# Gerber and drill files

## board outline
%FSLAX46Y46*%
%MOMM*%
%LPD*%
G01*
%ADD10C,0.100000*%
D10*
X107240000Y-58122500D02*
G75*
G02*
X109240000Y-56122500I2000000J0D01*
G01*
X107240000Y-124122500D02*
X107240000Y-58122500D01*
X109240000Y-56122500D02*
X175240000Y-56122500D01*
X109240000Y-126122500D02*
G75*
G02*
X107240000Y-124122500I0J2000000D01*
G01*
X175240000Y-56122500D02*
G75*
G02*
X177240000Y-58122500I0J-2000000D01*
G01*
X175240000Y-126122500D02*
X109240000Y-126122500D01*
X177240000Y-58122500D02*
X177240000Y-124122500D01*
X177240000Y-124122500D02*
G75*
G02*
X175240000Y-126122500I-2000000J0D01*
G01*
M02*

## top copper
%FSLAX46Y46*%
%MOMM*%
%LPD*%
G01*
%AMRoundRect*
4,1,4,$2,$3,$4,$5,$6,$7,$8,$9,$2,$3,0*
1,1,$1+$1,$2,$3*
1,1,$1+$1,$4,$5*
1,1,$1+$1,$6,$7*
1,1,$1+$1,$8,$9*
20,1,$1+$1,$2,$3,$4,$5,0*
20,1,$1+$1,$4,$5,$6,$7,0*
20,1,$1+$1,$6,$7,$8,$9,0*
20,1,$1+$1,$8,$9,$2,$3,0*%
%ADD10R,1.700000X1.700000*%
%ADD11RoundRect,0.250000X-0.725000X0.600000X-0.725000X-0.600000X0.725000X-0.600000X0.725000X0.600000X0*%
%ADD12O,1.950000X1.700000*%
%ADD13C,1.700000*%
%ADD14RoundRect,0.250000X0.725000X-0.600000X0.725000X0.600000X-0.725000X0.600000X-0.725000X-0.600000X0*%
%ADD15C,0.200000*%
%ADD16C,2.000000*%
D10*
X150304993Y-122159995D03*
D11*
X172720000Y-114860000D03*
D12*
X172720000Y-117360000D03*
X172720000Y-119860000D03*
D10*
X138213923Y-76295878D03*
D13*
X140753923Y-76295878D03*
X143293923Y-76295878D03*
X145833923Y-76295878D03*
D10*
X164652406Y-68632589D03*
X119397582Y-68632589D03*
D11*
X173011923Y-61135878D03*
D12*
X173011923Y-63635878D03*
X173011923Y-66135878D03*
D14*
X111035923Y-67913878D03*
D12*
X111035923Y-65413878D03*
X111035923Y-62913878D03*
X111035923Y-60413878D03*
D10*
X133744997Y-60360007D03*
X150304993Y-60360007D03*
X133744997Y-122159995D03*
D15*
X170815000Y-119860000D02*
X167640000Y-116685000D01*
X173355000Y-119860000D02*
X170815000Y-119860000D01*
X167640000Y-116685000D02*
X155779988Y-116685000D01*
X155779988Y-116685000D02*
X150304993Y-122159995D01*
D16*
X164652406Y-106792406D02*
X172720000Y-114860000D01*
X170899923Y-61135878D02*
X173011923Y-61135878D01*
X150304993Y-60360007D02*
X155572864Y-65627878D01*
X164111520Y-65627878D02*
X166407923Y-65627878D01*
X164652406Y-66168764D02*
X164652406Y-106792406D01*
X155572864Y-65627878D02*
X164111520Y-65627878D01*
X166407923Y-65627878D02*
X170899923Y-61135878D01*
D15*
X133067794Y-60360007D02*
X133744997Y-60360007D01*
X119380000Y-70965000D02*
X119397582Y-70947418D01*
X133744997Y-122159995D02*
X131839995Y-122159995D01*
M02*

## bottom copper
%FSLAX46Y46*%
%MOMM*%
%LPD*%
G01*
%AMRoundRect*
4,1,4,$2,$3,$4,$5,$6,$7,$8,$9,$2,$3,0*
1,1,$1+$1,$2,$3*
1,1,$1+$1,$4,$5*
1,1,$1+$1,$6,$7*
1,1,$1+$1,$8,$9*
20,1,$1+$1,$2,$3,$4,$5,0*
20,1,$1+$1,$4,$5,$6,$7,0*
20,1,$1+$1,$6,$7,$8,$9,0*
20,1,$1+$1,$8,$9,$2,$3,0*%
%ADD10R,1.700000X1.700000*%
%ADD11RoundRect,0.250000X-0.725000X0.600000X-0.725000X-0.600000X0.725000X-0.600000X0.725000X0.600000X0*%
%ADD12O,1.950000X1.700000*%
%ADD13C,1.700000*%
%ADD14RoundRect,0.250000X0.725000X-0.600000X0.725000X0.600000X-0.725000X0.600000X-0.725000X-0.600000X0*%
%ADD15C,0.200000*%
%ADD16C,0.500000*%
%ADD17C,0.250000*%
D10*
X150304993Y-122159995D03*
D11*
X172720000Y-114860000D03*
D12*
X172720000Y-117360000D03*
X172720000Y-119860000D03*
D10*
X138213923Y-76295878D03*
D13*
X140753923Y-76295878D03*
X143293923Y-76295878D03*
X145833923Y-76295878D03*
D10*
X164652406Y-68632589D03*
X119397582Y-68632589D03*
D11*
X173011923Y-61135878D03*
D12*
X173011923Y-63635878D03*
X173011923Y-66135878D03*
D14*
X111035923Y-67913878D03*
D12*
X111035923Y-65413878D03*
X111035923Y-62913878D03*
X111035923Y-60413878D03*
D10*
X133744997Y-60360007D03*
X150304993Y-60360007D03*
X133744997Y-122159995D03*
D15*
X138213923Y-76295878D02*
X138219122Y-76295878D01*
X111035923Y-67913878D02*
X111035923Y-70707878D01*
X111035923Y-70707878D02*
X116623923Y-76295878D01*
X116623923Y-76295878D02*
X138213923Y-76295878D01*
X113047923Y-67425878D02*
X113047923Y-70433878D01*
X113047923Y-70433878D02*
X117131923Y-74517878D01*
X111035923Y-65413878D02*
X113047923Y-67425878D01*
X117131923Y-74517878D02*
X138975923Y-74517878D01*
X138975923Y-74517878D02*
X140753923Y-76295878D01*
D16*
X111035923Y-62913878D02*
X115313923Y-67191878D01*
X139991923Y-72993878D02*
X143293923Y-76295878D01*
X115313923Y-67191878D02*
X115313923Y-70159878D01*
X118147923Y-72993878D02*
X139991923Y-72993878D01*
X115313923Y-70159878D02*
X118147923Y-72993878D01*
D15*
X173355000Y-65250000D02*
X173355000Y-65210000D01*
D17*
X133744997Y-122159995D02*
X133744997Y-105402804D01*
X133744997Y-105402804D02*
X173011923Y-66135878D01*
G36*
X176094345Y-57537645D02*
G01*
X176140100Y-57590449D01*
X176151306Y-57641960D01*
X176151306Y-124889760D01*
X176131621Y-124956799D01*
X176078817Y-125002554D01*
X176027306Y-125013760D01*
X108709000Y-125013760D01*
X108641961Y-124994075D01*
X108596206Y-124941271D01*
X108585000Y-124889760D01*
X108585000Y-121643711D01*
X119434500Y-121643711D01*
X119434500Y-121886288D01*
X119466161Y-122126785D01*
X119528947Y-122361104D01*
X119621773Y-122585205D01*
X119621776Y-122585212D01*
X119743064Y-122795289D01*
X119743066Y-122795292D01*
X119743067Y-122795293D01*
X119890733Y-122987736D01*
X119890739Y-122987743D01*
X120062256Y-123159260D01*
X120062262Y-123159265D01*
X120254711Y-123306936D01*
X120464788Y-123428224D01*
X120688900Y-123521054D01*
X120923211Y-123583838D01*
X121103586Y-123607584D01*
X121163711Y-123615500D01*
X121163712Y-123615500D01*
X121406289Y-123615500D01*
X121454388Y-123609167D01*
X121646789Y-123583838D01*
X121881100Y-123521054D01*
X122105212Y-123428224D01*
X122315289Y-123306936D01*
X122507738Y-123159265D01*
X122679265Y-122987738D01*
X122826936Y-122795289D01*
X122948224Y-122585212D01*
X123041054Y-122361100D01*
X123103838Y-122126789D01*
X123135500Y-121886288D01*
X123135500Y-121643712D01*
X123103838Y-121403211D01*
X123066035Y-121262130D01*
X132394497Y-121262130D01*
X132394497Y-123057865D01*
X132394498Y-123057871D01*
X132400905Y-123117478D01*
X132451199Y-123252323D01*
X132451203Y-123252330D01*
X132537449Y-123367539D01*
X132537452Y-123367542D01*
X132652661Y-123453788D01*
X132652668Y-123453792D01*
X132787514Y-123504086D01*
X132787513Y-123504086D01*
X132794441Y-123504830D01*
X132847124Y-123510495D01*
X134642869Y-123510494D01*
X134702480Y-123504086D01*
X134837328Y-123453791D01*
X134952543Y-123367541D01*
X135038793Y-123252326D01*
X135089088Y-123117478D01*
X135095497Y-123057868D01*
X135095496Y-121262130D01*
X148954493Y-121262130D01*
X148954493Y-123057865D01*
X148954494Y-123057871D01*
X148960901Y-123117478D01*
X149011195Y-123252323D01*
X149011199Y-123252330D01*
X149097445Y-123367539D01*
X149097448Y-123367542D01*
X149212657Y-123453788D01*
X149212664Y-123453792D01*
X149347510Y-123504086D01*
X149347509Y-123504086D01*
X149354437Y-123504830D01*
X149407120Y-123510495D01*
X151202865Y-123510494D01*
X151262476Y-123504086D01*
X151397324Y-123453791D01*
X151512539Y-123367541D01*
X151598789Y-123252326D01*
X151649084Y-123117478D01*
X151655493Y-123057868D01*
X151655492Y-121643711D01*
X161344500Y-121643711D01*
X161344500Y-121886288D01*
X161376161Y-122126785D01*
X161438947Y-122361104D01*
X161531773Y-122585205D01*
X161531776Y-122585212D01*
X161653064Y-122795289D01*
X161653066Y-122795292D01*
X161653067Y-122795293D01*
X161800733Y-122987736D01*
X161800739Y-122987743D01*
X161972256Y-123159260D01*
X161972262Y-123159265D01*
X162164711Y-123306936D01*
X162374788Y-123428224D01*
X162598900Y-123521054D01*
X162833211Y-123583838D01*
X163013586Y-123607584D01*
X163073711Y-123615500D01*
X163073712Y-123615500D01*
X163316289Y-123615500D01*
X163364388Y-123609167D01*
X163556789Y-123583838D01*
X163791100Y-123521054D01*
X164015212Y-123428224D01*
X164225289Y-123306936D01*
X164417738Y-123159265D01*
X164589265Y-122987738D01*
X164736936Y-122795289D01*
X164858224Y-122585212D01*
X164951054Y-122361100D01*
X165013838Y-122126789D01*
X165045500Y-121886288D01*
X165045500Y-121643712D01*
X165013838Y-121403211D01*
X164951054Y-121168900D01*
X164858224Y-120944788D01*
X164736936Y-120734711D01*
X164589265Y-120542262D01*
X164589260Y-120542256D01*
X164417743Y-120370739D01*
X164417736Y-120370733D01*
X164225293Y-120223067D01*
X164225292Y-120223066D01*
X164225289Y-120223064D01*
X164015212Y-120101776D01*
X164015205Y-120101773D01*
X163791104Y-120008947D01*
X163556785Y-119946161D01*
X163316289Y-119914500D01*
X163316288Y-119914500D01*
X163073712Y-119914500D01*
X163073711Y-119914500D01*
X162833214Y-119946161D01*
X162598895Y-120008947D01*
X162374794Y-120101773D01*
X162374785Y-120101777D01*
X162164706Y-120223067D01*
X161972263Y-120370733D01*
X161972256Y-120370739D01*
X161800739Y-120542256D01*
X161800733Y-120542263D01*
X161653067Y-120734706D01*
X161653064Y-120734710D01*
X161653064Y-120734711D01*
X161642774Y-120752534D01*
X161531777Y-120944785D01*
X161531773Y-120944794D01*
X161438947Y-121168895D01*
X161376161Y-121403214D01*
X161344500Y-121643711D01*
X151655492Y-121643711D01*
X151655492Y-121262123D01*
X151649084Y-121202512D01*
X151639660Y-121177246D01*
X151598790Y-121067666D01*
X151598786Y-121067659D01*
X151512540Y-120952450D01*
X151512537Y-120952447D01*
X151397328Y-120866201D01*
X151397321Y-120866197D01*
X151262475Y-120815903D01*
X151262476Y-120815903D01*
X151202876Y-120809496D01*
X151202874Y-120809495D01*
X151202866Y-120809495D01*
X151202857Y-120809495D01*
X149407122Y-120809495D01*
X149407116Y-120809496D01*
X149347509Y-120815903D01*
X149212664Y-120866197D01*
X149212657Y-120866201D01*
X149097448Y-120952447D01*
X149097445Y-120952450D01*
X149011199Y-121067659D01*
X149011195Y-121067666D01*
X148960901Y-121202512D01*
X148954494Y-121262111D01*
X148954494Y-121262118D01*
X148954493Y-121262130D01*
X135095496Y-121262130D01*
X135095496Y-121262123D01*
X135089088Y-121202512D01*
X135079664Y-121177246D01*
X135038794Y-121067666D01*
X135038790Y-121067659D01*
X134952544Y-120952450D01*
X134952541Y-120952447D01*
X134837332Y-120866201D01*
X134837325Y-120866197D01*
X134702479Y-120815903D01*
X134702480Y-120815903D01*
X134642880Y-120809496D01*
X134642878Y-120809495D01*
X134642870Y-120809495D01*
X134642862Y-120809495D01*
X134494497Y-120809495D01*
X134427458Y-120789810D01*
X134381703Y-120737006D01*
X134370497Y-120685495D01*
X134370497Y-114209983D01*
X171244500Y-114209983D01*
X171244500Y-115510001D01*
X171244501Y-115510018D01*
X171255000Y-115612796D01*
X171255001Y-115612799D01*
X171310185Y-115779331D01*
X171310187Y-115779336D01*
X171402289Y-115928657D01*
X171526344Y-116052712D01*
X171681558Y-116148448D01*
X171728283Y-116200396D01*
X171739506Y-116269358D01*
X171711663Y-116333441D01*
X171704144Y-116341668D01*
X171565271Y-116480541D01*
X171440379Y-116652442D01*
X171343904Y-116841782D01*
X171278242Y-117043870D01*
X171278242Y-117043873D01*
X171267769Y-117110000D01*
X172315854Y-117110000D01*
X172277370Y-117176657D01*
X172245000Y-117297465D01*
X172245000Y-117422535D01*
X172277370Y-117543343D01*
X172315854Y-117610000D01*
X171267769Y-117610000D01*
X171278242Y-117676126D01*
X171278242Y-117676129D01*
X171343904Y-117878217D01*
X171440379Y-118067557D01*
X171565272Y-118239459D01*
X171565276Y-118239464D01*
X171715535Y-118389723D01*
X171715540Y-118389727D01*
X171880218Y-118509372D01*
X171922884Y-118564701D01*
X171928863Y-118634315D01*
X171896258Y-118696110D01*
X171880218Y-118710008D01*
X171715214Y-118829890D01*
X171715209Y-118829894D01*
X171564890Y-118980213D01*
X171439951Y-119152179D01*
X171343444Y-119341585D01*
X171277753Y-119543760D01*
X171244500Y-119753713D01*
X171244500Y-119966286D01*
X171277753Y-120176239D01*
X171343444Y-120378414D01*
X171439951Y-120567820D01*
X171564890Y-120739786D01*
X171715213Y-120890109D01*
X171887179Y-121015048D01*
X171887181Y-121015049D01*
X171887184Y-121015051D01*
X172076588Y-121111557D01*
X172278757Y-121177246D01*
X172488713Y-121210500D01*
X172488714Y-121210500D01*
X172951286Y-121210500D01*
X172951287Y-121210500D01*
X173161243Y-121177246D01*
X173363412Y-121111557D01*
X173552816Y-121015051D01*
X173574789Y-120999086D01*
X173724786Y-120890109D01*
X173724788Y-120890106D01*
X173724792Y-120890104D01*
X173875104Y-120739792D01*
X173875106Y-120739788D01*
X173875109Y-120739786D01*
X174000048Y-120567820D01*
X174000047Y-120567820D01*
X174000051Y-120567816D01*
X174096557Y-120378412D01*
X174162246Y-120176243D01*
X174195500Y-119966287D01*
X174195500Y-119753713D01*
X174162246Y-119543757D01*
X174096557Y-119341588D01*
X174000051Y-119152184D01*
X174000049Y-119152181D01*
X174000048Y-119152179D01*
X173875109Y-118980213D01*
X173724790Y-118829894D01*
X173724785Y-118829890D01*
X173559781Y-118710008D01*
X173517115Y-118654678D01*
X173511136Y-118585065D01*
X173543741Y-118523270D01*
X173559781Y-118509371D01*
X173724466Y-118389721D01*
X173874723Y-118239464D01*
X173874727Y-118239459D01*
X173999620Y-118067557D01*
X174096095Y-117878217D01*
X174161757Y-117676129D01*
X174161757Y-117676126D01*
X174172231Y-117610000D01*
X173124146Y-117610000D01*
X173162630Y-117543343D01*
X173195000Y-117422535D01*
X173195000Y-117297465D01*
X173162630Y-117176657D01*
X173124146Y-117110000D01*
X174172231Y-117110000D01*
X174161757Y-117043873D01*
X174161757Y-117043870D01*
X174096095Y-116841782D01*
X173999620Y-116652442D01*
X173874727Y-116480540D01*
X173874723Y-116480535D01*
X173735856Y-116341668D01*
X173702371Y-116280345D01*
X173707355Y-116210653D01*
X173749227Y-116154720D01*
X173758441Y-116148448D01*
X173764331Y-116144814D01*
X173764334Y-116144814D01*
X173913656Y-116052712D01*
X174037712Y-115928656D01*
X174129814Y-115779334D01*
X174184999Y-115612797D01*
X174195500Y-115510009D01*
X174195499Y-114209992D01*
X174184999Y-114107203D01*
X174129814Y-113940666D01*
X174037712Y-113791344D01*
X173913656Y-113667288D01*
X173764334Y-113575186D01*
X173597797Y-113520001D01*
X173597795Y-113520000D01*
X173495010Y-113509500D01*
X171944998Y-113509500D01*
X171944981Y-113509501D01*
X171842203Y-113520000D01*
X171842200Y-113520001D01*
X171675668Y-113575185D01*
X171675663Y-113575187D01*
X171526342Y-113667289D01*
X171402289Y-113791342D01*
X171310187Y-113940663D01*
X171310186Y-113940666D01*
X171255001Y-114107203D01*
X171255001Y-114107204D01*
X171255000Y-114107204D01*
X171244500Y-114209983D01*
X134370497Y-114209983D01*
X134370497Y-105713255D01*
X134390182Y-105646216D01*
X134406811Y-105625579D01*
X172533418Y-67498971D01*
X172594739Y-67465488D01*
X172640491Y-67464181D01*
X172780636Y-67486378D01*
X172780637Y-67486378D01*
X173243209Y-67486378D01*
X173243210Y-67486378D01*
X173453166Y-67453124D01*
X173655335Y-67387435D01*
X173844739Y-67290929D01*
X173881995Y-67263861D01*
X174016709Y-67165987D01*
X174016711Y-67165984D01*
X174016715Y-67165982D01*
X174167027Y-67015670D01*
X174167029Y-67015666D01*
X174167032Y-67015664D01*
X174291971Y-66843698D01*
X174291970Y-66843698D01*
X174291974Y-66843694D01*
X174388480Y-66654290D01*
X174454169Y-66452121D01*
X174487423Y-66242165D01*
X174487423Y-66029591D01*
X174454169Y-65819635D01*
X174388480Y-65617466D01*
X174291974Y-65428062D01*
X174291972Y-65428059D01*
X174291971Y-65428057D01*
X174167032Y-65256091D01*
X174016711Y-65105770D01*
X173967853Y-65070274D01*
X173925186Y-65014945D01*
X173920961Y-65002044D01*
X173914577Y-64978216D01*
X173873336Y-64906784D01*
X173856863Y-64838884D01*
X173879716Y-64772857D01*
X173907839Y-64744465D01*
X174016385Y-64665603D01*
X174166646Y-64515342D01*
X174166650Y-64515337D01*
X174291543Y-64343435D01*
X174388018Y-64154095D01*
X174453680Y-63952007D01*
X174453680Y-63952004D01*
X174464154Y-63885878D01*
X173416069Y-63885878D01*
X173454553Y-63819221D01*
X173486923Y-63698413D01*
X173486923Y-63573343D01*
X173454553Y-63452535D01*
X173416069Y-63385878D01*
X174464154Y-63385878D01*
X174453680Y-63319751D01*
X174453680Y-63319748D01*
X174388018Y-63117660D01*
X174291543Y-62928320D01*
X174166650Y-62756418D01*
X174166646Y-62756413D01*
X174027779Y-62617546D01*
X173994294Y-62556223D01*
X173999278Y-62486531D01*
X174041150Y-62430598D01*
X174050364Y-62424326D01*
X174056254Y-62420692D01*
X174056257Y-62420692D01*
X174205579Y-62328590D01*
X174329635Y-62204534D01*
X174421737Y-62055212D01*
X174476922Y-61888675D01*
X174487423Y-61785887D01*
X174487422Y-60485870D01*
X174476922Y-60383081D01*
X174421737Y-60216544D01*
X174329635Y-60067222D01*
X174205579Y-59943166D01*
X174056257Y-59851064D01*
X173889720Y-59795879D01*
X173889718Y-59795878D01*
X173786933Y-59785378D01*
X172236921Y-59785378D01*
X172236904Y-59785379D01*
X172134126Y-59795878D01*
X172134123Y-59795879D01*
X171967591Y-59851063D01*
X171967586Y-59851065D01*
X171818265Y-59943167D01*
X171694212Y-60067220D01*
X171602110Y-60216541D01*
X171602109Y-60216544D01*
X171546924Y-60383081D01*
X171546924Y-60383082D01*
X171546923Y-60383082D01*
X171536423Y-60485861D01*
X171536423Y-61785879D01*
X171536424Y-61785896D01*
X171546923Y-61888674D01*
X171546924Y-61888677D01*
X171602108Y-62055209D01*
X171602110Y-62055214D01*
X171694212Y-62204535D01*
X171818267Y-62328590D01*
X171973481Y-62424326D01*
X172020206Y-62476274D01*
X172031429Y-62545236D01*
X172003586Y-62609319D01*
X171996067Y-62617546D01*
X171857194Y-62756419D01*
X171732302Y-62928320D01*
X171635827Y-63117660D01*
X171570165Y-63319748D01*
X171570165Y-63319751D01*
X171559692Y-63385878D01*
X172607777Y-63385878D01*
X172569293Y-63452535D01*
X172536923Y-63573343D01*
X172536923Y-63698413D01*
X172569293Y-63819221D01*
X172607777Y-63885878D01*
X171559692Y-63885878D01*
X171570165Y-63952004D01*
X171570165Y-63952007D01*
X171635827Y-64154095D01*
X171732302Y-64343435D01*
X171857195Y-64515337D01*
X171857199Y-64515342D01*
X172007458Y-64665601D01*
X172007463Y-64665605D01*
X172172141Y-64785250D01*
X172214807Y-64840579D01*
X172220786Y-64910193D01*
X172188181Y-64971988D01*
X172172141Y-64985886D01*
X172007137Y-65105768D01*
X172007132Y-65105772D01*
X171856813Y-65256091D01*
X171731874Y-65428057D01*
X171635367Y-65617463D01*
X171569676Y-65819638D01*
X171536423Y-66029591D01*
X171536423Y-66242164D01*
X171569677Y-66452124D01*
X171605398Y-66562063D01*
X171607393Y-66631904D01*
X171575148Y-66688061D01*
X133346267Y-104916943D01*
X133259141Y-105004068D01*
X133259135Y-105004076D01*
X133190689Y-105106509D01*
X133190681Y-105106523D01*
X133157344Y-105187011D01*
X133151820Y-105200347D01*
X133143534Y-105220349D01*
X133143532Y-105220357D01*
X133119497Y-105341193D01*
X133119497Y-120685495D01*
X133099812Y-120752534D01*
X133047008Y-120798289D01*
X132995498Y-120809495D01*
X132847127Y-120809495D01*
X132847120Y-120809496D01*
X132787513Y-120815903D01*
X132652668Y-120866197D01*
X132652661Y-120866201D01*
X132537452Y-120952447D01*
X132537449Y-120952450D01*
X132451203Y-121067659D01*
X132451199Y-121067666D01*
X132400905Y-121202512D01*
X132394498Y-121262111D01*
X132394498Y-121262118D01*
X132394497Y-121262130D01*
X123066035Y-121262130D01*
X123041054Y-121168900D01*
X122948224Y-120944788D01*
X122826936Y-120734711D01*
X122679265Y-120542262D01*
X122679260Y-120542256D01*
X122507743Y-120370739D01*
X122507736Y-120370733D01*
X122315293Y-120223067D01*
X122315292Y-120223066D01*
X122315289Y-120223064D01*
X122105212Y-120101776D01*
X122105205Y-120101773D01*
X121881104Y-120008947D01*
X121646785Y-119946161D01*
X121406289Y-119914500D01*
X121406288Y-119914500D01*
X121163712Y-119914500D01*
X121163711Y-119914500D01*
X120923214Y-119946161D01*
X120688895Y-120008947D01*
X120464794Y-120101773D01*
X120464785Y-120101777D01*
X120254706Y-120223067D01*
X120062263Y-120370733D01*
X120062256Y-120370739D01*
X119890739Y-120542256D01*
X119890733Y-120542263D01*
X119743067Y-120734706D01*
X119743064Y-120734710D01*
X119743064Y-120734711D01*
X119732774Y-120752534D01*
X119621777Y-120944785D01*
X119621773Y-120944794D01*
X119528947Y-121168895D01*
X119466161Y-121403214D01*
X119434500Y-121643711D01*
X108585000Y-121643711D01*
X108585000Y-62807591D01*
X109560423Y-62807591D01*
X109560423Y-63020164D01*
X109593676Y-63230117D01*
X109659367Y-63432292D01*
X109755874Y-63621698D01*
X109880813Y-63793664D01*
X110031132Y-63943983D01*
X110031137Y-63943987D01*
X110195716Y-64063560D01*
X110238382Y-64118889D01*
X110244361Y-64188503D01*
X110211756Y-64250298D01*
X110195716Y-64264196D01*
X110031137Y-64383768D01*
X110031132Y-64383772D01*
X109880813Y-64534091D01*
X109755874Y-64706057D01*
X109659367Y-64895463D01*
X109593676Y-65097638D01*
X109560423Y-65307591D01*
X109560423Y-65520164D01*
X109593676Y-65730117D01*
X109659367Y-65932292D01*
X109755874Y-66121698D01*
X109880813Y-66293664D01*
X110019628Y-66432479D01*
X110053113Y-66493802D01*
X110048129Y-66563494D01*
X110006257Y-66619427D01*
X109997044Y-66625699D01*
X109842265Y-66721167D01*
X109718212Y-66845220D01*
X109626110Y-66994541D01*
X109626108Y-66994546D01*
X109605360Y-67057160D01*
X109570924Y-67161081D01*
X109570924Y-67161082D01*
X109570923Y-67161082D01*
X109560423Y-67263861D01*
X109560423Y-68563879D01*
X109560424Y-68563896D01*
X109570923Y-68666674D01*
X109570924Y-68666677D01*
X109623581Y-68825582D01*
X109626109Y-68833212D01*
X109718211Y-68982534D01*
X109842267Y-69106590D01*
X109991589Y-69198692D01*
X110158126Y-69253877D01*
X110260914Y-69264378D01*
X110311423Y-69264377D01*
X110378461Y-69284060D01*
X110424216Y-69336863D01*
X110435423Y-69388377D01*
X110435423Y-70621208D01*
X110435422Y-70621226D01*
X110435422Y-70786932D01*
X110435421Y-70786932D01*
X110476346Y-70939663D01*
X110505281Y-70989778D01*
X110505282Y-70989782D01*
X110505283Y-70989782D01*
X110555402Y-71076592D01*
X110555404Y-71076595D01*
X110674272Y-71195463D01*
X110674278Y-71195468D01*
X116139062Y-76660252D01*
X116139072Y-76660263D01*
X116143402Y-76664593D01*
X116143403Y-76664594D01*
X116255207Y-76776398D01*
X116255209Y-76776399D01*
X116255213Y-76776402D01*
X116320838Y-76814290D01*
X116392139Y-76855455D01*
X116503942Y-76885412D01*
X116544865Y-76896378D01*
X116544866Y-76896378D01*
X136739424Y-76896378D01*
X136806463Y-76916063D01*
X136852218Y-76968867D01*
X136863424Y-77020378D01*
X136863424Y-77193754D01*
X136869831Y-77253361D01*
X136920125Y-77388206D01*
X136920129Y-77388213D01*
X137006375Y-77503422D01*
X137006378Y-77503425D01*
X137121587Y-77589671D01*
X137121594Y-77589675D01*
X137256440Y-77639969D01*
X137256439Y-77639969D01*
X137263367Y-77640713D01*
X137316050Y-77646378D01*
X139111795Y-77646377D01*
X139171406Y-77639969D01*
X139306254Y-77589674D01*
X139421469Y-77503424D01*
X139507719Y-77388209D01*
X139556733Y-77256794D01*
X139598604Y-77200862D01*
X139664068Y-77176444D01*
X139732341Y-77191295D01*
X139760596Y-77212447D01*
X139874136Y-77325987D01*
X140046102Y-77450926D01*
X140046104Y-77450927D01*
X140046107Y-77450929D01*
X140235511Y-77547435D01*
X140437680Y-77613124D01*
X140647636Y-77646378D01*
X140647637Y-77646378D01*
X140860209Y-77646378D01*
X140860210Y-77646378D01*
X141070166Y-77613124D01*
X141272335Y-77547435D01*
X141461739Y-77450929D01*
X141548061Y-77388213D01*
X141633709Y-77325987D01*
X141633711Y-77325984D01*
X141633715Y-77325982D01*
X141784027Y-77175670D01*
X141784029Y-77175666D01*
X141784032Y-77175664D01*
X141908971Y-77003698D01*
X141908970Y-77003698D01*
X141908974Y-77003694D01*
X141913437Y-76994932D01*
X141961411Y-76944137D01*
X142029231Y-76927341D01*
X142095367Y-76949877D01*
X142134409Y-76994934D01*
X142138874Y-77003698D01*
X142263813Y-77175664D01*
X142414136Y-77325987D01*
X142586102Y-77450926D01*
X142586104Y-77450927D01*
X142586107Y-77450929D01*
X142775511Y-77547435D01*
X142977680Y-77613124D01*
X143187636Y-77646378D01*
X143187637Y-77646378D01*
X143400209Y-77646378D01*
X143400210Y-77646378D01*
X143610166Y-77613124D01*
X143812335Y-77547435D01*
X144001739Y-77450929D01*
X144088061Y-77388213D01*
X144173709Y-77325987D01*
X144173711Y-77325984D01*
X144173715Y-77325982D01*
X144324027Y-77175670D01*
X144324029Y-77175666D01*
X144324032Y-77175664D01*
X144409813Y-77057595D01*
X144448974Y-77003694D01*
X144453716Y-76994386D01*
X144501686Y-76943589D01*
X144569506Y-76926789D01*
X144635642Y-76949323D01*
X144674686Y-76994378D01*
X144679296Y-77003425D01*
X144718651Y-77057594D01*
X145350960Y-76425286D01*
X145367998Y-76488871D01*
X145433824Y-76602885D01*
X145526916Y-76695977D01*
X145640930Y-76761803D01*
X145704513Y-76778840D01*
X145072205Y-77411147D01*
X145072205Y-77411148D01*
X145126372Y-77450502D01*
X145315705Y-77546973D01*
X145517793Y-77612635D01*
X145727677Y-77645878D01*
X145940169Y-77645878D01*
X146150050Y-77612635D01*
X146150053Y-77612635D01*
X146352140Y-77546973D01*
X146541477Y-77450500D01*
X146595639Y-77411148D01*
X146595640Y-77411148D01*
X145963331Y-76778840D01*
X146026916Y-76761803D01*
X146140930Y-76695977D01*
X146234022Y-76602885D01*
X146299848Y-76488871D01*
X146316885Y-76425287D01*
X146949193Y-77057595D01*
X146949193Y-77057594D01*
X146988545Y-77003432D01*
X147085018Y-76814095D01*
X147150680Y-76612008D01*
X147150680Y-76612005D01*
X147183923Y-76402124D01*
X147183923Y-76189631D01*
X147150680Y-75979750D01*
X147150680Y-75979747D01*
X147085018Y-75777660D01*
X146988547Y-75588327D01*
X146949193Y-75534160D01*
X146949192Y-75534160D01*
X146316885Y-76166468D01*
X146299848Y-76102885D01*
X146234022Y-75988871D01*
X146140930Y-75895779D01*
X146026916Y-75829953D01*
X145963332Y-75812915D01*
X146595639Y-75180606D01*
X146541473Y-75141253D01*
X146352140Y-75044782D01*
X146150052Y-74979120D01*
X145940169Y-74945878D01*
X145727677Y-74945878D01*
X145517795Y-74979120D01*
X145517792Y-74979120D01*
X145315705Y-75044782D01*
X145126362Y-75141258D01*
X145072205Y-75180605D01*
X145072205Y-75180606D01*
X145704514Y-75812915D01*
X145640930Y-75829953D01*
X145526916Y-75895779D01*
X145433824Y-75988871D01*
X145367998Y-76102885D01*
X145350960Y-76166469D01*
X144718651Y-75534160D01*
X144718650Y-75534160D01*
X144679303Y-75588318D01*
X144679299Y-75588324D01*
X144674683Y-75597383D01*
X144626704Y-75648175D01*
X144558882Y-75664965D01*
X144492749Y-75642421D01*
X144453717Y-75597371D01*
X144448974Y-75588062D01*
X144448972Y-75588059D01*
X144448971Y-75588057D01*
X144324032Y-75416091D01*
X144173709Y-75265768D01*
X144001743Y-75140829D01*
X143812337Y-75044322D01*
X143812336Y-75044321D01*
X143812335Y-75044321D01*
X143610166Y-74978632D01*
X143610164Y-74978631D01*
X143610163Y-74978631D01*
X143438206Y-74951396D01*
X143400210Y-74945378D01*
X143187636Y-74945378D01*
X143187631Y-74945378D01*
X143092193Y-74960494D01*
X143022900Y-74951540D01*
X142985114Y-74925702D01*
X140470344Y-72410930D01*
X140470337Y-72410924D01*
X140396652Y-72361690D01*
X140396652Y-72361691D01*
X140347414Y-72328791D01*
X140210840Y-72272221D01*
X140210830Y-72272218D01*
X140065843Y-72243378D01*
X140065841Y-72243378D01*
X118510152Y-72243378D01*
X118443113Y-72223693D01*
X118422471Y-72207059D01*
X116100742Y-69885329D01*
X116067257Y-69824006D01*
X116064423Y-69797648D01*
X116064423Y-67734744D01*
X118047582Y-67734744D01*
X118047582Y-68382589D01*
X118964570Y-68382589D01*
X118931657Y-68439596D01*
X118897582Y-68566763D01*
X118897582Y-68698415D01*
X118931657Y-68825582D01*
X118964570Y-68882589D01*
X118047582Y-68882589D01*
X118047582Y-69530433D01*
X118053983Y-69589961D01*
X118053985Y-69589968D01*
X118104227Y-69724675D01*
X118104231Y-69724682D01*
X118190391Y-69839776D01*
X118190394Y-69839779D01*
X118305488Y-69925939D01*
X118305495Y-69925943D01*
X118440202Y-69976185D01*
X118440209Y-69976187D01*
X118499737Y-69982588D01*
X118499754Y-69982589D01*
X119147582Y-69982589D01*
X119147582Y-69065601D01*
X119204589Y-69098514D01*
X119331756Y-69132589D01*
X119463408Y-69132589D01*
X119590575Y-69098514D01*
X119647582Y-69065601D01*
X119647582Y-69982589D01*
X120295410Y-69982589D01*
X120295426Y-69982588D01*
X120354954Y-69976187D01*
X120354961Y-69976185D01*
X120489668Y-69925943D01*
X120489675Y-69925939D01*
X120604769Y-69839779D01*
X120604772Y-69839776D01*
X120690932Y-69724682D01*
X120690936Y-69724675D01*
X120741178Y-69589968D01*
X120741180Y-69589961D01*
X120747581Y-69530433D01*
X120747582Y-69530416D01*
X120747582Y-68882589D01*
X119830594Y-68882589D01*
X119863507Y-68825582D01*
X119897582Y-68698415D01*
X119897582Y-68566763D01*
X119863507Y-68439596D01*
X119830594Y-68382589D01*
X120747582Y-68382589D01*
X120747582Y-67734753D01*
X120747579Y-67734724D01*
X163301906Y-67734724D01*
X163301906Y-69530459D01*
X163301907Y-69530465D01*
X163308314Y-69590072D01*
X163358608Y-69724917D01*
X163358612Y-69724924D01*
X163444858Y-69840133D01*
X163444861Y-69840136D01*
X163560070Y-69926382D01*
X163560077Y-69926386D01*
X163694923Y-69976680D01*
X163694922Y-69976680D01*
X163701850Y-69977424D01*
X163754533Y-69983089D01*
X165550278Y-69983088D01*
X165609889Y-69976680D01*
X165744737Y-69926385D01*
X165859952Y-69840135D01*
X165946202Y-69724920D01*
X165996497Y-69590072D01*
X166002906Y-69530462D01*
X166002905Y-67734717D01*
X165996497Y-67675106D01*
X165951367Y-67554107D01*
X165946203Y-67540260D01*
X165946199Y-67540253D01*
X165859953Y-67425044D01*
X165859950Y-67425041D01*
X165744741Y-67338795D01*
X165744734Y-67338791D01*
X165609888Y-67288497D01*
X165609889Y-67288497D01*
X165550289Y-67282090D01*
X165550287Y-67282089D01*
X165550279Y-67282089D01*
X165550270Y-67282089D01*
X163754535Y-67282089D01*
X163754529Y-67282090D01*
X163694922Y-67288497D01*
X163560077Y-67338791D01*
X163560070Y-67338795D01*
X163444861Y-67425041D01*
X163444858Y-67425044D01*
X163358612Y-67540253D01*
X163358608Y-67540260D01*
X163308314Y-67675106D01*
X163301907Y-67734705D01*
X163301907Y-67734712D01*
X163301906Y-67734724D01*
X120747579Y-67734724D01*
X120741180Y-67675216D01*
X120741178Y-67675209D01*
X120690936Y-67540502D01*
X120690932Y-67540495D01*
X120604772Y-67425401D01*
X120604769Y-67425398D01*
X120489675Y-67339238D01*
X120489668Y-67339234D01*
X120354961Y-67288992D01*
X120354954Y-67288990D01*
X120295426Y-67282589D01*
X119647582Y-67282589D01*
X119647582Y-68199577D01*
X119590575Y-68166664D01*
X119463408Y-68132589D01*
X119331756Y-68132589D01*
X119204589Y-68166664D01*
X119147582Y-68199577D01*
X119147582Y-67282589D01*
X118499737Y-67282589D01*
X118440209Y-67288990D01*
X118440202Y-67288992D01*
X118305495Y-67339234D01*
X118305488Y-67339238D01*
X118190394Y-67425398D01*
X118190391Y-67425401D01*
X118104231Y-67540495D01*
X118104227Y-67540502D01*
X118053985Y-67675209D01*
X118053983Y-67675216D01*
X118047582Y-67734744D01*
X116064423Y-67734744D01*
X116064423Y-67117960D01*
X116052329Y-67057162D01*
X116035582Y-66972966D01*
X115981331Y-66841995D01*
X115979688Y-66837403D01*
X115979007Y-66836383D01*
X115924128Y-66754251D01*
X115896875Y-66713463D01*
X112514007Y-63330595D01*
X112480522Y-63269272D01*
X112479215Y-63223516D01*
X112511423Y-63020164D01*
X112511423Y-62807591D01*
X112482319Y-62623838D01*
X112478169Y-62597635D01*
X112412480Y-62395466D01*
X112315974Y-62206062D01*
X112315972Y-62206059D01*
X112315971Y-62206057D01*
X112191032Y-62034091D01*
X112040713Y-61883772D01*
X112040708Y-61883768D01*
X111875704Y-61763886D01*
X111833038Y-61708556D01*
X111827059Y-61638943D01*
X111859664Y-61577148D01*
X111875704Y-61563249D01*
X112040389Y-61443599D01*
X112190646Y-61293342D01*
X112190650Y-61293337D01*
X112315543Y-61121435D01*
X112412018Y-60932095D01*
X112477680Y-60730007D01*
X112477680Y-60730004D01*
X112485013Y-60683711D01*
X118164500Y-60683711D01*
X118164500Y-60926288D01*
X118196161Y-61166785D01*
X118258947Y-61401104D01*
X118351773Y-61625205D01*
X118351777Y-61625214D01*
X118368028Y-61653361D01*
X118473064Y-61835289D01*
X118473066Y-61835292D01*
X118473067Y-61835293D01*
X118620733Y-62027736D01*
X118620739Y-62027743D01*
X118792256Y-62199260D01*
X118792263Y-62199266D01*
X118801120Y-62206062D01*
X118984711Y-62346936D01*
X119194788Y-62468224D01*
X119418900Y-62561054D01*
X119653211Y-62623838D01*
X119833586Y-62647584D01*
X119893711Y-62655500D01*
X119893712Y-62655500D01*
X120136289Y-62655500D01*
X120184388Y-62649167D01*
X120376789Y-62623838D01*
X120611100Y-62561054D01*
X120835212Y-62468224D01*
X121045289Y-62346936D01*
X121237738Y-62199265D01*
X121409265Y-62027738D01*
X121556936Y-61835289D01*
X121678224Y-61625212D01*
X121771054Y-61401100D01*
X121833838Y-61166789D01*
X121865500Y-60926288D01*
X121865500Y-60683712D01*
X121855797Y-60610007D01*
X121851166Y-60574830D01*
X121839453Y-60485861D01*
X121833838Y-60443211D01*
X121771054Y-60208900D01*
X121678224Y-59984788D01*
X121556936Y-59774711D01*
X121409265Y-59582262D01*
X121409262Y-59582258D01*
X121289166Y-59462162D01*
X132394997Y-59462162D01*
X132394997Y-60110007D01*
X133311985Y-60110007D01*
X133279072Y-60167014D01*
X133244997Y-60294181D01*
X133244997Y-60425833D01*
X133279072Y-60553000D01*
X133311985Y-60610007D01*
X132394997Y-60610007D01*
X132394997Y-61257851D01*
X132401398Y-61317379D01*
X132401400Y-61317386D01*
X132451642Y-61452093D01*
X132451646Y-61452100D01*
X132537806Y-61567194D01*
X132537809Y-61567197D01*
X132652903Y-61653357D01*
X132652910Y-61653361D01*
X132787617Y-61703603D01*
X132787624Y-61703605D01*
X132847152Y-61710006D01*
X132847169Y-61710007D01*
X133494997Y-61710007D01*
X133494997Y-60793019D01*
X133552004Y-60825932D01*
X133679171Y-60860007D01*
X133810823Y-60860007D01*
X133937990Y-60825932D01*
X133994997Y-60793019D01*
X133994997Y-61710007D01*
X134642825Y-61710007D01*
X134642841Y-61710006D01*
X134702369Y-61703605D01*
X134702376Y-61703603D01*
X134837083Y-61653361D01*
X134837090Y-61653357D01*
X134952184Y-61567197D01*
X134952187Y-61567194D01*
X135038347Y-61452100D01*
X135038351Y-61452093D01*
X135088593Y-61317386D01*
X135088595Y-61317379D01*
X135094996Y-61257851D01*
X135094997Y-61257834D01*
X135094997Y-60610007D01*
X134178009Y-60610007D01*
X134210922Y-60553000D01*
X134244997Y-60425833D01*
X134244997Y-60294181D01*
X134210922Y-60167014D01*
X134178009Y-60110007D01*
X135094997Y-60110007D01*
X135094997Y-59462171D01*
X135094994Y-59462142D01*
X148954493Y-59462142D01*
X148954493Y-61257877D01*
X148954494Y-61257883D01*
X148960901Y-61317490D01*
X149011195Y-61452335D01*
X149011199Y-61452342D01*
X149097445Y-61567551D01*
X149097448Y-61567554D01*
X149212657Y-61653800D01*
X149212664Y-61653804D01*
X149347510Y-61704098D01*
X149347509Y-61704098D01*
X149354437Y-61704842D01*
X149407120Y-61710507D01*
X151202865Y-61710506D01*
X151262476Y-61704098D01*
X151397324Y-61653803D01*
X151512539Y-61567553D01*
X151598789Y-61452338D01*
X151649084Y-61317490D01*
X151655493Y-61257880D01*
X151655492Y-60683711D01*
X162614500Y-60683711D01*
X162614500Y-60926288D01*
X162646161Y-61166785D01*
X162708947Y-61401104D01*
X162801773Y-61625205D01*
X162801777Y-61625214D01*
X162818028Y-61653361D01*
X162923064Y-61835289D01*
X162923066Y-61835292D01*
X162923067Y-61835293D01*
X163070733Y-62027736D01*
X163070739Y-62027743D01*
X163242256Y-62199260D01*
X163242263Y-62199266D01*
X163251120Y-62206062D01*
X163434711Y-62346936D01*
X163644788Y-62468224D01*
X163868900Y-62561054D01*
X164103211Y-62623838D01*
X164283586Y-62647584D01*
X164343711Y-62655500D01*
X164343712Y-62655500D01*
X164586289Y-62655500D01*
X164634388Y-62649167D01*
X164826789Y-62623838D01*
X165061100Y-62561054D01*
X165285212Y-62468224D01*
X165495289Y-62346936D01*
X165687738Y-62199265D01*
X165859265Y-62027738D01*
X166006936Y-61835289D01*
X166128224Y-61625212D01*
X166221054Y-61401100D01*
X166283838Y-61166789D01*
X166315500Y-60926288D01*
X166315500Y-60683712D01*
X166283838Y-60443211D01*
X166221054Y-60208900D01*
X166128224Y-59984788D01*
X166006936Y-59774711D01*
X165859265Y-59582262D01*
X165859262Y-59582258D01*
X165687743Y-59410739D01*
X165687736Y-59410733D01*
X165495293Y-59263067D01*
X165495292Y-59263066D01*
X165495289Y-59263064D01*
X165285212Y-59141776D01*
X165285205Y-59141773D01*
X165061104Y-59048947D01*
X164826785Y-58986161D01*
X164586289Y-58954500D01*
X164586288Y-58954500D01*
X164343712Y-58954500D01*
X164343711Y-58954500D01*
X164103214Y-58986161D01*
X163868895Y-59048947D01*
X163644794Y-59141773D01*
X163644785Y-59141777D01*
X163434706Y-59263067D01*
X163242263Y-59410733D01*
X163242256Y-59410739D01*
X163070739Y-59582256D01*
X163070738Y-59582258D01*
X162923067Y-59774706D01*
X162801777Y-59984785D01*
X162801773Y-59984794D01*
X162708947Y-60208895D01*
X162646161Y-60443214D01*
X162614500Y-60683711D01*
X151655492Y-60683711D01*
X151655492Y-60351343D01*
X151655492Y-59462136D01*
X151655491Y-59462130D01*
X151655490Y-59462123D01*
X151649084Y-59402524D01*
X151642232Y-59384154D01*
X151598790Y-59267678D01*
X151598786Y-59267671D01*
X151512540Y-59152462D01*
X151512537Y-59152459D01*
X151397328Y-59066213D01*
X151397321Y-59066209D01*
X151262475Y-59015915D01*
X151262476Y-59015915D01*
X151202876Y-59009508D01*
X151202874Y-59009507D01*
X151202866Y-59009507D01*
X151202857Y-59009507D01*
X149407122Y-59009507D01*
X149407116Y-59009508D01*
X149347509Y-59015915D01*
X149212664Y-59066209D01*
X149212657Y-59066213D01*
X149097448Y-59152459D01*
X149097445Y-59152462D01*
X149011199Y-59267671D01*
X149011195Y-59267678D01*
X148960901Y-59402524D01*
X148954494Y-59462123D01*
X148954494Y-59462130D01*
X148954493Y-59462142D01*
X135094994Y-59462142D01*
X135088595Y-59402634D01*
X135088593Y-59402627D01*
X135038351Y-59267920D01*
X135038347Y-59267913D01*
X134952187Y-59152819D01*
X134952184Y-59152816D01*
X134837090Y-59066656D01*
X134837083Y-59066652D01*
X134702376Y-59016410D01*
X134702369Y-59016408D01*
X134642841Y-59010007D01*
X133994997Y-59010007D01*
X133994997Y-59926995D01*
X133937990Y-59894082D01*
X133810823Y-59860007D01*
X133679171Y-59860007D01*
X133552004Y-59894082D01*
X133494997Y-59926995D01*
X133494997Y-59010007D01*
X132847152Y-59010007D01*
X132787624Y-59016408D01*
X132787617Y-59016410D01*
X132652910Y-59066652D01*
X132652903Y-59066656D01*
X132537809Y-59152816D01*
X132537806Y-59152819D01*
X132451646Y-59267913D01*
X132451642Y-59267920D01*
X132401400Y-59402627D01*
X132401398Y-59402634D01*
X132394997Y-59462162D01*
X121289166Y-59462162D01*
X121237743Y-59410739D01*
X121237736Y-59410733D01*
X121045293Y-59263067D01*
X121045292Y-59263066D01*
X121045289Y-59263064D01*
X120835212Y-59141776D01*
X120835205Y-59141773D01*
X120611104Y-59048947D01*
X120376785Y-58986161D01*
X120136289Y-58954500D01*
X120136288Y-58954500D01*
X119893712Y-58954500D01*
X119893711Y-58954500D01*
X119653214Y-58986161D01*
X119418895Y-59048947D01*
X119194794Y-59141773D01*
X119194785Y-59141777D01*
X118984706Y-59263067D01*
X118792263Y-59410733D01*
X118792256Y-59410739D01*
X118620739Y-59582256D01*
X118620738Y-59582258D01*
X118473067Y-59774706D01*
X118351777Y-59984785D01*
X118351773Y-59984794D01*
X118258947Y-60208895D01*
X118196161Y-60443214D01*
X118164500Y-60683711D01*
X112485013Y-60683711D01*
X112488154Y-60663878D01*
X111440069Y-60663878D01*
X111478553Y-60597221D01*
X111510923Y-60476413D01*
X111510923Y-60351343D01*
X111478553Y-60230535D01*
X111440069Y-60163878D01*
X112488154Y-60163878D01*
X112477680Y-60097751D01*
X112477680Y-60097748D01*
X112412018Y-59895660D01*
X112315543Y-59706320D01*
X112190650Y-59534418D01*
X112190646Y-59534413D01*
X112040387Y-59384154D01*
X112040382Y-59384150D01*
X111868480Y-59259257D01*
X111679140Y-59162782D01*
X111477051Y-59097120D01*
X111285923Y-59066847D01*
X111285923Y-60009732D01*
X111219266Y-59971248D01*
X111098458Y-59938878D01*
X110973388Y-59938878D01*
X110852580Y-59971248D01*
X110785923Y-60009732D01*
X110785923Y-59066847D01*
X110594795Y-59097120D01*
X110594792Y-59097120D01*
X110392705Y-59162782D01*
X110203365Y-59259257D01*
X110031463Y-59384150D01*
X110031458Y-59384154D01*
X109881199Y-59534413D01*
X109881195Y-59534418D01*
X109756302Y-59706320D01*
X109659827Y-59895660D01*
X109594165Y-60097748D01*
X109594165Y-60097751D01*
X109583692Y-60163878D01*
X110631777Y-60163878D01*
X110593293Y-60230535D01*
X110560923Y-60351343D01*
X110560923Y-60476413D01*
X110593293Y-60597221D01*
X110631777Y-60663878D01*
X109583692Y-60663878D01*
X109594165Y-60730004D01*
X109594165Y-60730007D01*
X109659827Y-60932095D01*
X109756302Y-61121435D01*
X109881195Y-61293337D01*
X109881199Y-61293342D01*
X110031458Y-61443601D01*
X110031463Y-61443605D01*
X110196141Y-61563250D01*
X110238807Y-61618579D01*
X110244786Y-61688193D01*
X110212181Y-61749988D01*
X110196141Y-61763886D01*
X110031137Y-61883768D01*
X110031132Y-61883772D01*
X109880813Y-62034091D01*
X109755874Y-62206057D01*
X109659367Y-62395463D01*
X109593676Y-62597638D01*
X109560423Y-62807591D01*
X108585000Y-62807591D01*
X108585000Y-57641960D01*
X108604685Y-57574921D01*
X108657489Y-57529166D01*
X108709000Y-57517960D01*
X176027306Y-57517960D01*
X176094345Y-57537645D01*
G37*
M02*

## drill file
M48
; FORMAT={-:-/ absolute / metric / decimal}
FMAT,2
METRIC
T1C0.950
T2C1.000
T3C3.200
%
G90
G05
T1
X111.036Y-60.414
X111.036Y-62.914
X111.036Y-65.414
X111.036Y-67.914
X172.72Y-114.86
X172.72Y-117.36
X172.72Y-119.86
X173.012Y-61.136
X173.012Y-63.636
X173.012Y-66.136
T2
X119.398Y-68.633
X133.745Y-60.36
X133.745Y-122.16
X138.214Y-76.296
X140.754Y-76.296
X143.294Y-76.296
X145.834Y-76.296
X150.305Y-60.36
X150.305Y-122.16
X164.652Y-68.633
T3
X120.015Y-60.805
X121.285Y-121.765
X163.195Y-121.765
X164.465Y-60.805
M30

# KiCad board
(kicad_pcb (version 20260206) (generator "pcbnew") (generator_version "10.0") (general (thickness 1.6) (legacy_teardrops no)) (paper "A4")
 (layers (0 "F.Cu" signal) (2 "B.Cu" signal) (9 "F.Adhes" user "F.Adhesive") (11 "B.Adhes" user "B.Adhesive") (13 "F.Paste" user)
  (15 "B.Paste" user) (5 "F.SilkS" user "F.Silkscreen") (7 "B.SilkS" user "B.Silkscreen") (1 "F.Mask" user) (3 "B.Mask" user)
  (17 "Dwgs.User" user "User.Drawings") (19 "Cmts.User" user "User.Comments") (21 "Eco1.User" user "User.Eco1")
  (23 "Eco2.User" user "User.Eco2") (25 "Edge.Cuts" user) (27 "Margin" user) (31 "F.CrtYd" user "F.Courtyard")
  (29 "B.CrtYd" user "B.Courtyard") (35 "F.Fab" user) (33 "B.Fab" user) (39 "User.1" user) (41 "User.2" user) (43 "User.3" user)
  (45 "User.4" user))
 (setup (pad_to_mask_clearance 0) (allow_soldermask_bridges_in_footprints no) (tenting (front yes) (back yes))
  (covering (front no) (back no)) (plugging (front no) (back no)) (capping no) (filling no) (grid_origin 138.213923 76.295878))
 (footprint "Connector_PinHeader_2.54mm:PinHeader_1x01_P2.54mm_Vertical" (layer "F.Cu") (at 150.304993 122.159995)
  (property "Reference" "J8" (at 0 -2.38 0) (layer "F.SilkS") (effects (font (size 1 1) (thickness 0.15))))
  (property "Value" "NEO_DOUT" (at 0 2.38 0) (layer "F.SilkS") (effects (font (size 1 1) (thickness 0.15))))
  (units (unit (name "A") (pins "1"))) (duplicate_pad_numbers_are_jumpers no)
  (pad "1" thru_hole rect (at 0 0) (size 1.7 1.7) (drill 1) (layers "*.Cu" "*.Mask") (remove_unused_layers no) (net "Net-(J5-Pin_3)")))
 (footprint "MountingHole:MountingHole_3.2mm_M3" (layer "F.Cu") (at 163.195 121.765)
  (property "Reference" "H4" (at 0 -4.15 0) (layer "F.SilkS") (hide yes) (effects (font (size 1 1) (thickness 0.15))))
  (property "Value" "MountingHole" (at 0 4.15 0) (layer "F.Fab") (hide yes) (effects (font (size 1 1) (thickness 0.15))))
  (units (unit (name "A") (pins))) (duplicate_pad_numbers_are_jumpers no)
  (pad "" np_thru_hole circle (at 0 0) (size 3.2 3.2) (drill 3.2) (layers "*.Cu" "*.Mask")))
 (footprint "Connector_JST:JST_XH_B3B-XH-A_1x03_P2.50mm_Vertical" (layer "F.Cu") (at 172.72 114.86 -90)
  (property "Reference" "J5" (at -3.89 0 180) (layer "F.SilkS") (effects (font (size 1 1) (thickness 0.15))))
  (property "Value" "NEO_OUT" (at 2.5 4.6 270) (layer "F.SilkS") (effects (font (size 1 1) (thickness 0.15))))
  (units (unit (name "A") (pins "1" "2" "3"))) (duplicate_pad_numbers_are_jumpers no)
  (pad "1" thru_hole roundrect (at 0 0 270) (size 1.7 1.95) (drill 0.95) (layers "*.Cu" "*.Mask") (remove_unused_layers no)
   (roundrect_rratio 0.147059) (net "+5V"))
  (pad "2" thru_hole oval (at 2.5 0 270) (size 1.7 1.95) (drill 0.95) (layers "*.Cu" "*.Mask") (remove_unused_layers no) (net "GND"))
  (pad "3" thru_hole oval (at 5 0 270) (size 1.7 1.95) (drill 0.95) (layers "*.Cu" "*.Mask") (remove_unused_layers no)
   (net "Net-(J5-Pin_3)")))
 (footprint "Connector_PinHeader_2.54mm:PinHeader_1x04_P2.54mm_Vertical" (layer "F.Cu") (at 138.213923 76.295878 90)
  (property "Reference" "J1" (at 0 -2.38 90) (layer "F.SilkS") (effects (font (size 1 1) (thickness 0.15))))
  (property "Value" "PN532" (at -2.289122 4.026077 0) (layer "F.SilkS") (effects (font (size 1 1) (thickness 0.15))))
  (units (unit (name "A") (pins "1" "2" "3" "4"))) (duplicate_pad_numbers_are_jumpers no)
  (pad "1" thru_hole rect (at 0 0 90) (size 1.7 1.7) (drill 1) (layers "*.Cu" "*.Mask") (remove_unused_layers no) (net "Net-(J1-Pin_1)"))
  (pad "2" thru_hole circle (at 0 2.54 90) (size 1.7 1.7) (drill 1) (layers "*.Cu" "*.Mask") (remove_unused_layers no)
   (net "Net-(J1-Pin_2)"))
  (pad "3" thru_hole circle (at 0 5.08 90) (size 1.7 1.7) (drill 1) (layers "*.Cu" "*.Mask") (remove_unused_layers no)
   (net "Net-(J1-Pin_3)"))
  (pad "4" thru_hole circle (at 0 7.62 90) (size 1.7 1.7) (drill 1) (layers "*.Cu" "*.Mask") (remove_unused_layers no) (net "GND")))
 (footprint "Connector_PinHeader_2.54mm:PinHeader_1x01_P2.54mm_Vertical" (layer "F.Cu") (at 164.652406 68.632589)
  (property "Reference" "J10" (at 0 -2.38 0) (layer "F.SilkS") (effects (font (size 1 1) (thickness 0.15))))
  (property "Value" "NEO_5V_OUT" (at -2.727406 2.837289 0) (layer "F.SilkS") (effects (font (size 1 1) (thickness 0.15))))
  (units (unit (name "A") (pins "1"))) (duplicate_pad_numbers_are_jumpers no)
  (pad "1" thru_hole rect (at 0 0) (size 1.7 1.7) (drill 1) (layers "*.Cu" "*.Mask") (remove_unused_layers no) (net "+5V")))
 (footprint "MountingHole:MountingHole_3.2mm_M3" (layer "F.Cu") (at 121.285 121.765)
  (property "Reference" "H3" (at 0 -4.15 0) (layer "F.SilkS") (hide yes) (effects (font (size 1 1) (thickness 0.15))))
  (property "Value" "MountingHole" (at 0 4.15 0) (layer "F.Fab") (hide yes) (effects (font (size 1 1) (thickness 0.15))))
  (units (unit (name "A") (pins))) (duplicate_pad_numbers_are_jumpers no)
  (pad "" np_thru_hole circle (at 0 0) (size 3.2 3.2) (drill 3.2) (layers "*.Cu" "*.Mask")))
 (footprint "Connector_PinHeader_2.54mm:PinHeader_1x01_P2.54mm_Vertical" (layer "F.Cu") (at 119.397582 68.632589)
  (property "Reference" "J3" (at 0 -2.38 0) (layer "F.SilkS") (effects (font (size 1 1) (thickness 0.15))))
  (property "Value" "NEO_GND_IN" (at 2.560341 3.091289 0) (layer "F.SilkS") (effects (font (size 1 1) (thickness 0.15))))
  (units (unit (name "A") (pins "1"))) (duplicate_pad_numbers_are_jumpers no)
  (pad "1" thru_hole rect (at 0 0) (size 1.7 1.7) (drill 1) (layers "*.Cu" "*.Mask") (remove_unused_layers no) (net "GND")))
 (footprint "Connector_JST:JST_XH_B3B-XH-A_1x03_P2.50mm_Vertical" (layer "F.Cu") (at 173.011923 61.135878 -90)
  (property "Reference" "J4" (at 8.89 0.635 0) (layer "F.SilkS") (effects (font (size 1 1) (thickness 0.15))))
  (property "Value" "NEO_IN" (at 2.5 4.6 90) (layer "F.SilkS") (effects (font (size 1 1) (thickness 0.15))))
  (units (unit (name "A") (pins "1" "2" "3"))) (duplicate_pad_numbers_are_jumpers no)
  (pad "1" thru_hole roundrect (at 0 0 270) (size 1.7 1.95) (drill 0.95) (layers "*.Cu" "*.Mask") (remove_unused_layers no)
   (roundrect_rratio 0.147059) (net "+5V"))
  (pad "2" thru_hole oval (at 2.5 0 270) (size 1.7 1.95) (drill 0.95) (layers "*.Cu" "*.Mask") (remove_unused_layers no) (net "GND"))
  (pad "3" thru_hole oval (at 5 0 270) (size 1.7 1.95) (drill 0.95) (layers "*.Cu" "*.Mask") (remove_unused_layers no)
   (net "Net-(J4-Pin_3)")))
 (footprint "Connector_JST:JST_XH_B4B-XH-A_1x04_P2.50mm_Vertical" (layer "F.Cu") (at 111.035923 67.913878 90)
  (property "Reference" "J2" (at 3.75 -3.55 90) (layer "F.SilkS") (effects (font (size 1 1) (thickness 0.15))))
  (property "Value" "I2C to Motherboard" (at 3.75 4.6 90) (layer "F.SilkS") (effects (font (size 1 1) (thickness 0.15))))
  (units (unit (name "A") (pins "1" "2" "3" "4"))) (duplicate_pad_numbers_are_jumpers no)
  (pad "1" thru_hole roundrect (at 0 0 90) (size 1.7 1.95) (drill 0.95) (layers "*.Cu" "*.Mask") (remove_unused_layers no)
   (roundrect_rratio 0.147059) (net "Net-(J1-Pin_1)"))
  (pad "2" thru_hole oval (at 2.5 0 90) (size 1.7 1.95) (drill 0.95) (layers "*.Cu" "*.Mask") (remove_unused_layers no)
   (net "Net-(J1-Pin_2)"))
  (pad "3" thru_hole oval (at 5 0 90) (size 1.7 1.95) (drill 0.95) (layers "*.Cu" "*.Mask") (remove_unused_layers no) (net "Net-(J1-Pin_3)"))
  (pad "4" thru_hole oval (at 7.5 0 90) (size 1.7 1.95) (drill 0.95) (layers "*.Cu" "*.Mask") (remove_unused_layers no) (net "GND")))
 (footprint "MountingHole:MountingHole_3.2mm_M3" (layer "F.Cu") (at 120.015 60.805)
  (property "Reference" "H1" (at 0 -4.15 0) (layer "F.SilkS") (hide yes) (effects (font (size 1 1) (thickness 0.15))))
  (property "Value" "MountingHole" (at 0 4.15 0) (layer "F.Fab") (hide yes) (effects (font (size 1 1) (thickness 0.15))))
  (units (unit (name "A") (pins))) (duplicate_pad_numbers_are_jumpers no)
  (pad "" np_thru_hole circle (at 0 0) (size 3.2 3.2) (drill 3.2) (layers "*.Cu" "*.Mask")))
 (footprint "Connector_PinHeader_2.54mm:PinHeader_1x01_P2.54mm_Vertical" (layer "F.Cu") (at 133.744997 60.360007)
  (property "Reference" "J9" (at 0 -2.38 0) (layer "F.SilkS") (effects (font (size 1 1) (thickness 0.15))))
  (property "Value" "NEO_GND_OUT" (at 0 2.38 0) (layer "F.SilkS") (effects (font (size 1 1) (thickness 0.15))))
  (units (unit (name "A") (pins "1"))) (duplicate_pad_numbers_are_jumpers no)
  (pad "1" thru_hole rect (at 0 0) (size 1.7 1.7) (drill 1) (layers "*.Cu" "*.Mask") (remove_unused_layers no) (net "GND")))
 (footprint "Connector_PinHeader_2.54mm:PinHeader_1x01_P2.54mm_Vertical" (layer "F.Cu") (at 150.304993 60.360007)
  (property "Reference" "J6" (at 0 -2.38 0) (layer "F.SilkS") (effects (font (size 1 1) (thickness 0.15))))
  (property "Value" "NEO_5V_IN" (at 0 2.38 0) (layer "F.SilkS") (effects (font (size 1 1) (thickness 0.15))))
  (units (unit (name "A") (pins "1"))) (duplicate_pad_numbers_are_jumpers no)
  (pad "1" thru_hole rect (at 0 0) (size 1.7 1.7) (drill 1) (layers "*.Cu" "*.Mask") (remove_unused_layers no) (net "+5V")))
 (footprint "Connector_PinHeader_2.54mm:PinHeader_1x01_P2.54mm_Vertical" (layer "F.Cu") (at 133.744997 122.159995)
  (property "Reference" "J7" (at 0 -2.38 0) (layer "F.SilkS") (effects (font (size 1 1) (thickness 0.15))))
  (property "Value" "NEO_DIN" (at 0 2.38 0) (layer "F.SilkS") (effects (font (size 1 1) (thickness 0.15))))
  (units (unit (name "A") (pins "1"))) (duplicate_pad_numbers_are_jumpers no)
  (pad "1" thru_hole rect (at 0 0) (size 1.7 1.7) (drill 1) (layers "*.Cu" "*.Mask") (remove_unused_layers no) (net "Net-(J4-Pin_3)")))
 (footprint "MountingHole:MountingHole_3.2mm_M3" (layer "F.Cu") (at 164.465 60.805)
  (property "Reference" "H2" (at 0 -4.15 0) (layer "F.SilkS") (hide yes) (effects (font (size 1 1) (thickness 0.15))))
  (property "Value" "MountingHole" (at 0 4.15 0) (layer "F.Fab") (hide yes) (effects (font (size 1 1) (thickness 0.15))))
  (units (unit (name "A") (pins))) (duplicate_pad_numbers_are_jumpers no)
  (pad "" np_thru_hole circle (at 0 0) (size 3.2 3.2) (drill 3.2) (layers "*.Cu" "*.Mask")))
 (gr_arc (start 107.24 58.1225) (mid 107.825786 56.708286) (end 109.24 56.1225) (stroke (width 0.1) (type default)) (layer "Edge.Cuts"))
 (gr_line (start 107.24 124.1225) (end 107.24 58.1225) (stroke (width 0.1) (type default)) (layer "Edge.Cuts"))
 (gr_line (start 109.24 56.1225) (end 175.24 56.1225) (stroke (width 0.1) (type default)) (layer "Edge.Cuts"))
 (gr_arc (start 109.24 126.1225) (mid 107.825786 125.536714) (end 107.24 124.1225) (stroke (width 0.1) (type default)) (layer "Edge.Cuts"))
 (gr_arc (start 175.24 56.1225) (mid 176.654214 56.708286) (end 177.24 58.1225) (stroke (width 0.1) (type default)) (layer "Edge.Cuts"))
 (gr_line (start 175.24 126.1225) (end 109.24 126.1225) (stroke (width 0.1) (type default)) (layer "Edge.Cuts"))
 (gr_line (start 177.24 58.1225) (end 177.24 124.1225) (stroke (width 0.1) (type default)) (layer "Edge.Cuts"))
 (gr_arc (start 177.24 124.1225) (mid 176.654214 125.536714) (end 175.24 126.1225) (stroke (width 0.1) (type default)) (layer "Edge.Cuts"))
 (segment (start 170.815 119.86) (end 167.64 116.685) (width 0.2) (layer "F.Cu") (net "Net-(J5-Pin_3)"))
 (segment (start 173.355 119.86) (end 170.815 119.86) (width 0.2) (layer "F.Cu") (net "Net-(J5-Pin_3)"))
 (segment (start 167.64 116.685) (end 155.779988 116.685) (width 0.2) (layer "F.Cu") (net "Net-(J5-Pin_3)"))
 (segment (start 155.779988 116.685) (end 150.304993 122.159995) (width 0.2) (layer "F.Cu") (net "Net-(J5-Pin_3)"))
 (segment (start 164.652406 106.792406) (end 172.72 114.86) (width 2) (layer "F.Cu") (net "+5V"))
 (segment (start 170.899923 61.135878) (end 173.011923 61.135878) (width 2) (layer "F.Cu") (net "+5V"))
 (segment (start 150.304993 60.360007) (end 155.572864 65.627878) (width 2) (layer "F.Cu") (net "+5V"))
 (segment (start 164.11152 65.627878) (end 166.407923 65.627878) (width 2) (layer "F.Cu") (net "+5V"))
 (segment (start 164.652406 66.168764) (end 164.652406 106.792406) (width 2) (layer "F.Cu") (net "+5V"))
 (segment (start 155.572864 65.627878) (end 164.11152 65.627878) (width 2) (layer "F.Cu") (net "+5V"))
 (segment (start 166.407923 65.627878) (end 170.899923 61.135878) (width 2) (layer "F.Cu") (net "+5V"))
 (segment (start 133.067794 60.360007) (end 133.744997 60.360007) (width 0.2) (layer "F.Cu") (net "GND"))
 (segment (start 119.38 70.965) (end 119.397582 70.947418) (width 0.2) (layer "F.Cu") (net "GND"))
 (segment (start 138.213923 76.295878) (end 138.219122 76.295878) (width 0.2) (layer "B.Cu") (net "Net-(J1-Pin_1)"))
 (segment (start 111.035923 67.913878) (end 111.035923 70.707878) (width 0.2) (layer "B.Cu") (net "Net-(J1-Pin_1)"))
 (segment (start 111.035923 70.707878) (end 116.623923 76.295878) (width 0.2) (layer "B.Cu") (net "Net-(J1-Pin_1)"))
 (segment (start 116.623923 76.295878) (end 138.213923 76.295878) (width 0.2) (layer "B.Cu") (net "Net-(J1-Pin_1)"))
 (segment (start 113.047923 67.425878) (end 113.047923 70.433878) (width 0.2) (layer "B.Cu") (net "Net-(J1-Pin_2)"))
 (segment (start 113.047923 70.433878) (end 117.131923 74.517878) (width 0.2) (layer "B.Cu") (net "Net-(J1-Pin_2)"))
 (segment (start 111.035923 65.413878) (end 113.047923 67.425878) (width 0.2) (layer "B.Cu") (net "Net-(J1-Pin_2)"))
 (segment (start 117.131923 74.517878) (end 138.975923 74.517878) (width 0.2) (layer "B.Cu") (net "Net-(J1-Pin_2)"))
 (segment (start 138.975923 74.517878) (end 140.753923 76.295878) (width 0.2) (layer "B.Cu") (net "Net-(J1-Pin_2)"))
 (segment (start 111.035923 62.913878) (end 115.313923 67.191878) (width 0.5) (layer "B.Cu") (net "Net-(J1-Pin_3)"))
 (segment (start 139.991923 72.993878) (end 143.293923 76.295878) (width 0.5) (layer "B.Cu") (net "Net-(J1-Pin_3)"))
 (segment (start 115.313923 67.191878) (end 115.313923 70.159878) (width 0.5) (layer "B.Cu") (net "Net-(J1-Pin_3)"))
 (segment (start 118.147923 72.993878) (end 139.991923 72.993878) (width 0.5) (layer "B.Cu") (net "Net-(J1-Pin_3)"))
 (segment (start 115.313923 70.159878) (end 118.147923 72.993878) (width 0.5) (layer "B.Cu") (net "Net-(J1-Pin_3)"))
 (segment (start 133.744997 122.159995) (end 131.839995 122.159995) (width 0.2) (layer "F.Cu") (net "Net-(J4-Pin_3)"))
 (segment (start 173.355 65.25) (end 173.355 65.21) (width 0.2) (layer "B.Cu") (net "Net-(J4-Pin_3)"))
 (segment (start 133.744997 122.159995) (end 133.744997 105.402804) (width 0.25) (layer "B.Cu") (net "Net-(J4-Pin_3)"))
 (segment (start 133.744997 105.402804) (end 173.011923 66.135878) (width 0.25) (layer "B.Cu") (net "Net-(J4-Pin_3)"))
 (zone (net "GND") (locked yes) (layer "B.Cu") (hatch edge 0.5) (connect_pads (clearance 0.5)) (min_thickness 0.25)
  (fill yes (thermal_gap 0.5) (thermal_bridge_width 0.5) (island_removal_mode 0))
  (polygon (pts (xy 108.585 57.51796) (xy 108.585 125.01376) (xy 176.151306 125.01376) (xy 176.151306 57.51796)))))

